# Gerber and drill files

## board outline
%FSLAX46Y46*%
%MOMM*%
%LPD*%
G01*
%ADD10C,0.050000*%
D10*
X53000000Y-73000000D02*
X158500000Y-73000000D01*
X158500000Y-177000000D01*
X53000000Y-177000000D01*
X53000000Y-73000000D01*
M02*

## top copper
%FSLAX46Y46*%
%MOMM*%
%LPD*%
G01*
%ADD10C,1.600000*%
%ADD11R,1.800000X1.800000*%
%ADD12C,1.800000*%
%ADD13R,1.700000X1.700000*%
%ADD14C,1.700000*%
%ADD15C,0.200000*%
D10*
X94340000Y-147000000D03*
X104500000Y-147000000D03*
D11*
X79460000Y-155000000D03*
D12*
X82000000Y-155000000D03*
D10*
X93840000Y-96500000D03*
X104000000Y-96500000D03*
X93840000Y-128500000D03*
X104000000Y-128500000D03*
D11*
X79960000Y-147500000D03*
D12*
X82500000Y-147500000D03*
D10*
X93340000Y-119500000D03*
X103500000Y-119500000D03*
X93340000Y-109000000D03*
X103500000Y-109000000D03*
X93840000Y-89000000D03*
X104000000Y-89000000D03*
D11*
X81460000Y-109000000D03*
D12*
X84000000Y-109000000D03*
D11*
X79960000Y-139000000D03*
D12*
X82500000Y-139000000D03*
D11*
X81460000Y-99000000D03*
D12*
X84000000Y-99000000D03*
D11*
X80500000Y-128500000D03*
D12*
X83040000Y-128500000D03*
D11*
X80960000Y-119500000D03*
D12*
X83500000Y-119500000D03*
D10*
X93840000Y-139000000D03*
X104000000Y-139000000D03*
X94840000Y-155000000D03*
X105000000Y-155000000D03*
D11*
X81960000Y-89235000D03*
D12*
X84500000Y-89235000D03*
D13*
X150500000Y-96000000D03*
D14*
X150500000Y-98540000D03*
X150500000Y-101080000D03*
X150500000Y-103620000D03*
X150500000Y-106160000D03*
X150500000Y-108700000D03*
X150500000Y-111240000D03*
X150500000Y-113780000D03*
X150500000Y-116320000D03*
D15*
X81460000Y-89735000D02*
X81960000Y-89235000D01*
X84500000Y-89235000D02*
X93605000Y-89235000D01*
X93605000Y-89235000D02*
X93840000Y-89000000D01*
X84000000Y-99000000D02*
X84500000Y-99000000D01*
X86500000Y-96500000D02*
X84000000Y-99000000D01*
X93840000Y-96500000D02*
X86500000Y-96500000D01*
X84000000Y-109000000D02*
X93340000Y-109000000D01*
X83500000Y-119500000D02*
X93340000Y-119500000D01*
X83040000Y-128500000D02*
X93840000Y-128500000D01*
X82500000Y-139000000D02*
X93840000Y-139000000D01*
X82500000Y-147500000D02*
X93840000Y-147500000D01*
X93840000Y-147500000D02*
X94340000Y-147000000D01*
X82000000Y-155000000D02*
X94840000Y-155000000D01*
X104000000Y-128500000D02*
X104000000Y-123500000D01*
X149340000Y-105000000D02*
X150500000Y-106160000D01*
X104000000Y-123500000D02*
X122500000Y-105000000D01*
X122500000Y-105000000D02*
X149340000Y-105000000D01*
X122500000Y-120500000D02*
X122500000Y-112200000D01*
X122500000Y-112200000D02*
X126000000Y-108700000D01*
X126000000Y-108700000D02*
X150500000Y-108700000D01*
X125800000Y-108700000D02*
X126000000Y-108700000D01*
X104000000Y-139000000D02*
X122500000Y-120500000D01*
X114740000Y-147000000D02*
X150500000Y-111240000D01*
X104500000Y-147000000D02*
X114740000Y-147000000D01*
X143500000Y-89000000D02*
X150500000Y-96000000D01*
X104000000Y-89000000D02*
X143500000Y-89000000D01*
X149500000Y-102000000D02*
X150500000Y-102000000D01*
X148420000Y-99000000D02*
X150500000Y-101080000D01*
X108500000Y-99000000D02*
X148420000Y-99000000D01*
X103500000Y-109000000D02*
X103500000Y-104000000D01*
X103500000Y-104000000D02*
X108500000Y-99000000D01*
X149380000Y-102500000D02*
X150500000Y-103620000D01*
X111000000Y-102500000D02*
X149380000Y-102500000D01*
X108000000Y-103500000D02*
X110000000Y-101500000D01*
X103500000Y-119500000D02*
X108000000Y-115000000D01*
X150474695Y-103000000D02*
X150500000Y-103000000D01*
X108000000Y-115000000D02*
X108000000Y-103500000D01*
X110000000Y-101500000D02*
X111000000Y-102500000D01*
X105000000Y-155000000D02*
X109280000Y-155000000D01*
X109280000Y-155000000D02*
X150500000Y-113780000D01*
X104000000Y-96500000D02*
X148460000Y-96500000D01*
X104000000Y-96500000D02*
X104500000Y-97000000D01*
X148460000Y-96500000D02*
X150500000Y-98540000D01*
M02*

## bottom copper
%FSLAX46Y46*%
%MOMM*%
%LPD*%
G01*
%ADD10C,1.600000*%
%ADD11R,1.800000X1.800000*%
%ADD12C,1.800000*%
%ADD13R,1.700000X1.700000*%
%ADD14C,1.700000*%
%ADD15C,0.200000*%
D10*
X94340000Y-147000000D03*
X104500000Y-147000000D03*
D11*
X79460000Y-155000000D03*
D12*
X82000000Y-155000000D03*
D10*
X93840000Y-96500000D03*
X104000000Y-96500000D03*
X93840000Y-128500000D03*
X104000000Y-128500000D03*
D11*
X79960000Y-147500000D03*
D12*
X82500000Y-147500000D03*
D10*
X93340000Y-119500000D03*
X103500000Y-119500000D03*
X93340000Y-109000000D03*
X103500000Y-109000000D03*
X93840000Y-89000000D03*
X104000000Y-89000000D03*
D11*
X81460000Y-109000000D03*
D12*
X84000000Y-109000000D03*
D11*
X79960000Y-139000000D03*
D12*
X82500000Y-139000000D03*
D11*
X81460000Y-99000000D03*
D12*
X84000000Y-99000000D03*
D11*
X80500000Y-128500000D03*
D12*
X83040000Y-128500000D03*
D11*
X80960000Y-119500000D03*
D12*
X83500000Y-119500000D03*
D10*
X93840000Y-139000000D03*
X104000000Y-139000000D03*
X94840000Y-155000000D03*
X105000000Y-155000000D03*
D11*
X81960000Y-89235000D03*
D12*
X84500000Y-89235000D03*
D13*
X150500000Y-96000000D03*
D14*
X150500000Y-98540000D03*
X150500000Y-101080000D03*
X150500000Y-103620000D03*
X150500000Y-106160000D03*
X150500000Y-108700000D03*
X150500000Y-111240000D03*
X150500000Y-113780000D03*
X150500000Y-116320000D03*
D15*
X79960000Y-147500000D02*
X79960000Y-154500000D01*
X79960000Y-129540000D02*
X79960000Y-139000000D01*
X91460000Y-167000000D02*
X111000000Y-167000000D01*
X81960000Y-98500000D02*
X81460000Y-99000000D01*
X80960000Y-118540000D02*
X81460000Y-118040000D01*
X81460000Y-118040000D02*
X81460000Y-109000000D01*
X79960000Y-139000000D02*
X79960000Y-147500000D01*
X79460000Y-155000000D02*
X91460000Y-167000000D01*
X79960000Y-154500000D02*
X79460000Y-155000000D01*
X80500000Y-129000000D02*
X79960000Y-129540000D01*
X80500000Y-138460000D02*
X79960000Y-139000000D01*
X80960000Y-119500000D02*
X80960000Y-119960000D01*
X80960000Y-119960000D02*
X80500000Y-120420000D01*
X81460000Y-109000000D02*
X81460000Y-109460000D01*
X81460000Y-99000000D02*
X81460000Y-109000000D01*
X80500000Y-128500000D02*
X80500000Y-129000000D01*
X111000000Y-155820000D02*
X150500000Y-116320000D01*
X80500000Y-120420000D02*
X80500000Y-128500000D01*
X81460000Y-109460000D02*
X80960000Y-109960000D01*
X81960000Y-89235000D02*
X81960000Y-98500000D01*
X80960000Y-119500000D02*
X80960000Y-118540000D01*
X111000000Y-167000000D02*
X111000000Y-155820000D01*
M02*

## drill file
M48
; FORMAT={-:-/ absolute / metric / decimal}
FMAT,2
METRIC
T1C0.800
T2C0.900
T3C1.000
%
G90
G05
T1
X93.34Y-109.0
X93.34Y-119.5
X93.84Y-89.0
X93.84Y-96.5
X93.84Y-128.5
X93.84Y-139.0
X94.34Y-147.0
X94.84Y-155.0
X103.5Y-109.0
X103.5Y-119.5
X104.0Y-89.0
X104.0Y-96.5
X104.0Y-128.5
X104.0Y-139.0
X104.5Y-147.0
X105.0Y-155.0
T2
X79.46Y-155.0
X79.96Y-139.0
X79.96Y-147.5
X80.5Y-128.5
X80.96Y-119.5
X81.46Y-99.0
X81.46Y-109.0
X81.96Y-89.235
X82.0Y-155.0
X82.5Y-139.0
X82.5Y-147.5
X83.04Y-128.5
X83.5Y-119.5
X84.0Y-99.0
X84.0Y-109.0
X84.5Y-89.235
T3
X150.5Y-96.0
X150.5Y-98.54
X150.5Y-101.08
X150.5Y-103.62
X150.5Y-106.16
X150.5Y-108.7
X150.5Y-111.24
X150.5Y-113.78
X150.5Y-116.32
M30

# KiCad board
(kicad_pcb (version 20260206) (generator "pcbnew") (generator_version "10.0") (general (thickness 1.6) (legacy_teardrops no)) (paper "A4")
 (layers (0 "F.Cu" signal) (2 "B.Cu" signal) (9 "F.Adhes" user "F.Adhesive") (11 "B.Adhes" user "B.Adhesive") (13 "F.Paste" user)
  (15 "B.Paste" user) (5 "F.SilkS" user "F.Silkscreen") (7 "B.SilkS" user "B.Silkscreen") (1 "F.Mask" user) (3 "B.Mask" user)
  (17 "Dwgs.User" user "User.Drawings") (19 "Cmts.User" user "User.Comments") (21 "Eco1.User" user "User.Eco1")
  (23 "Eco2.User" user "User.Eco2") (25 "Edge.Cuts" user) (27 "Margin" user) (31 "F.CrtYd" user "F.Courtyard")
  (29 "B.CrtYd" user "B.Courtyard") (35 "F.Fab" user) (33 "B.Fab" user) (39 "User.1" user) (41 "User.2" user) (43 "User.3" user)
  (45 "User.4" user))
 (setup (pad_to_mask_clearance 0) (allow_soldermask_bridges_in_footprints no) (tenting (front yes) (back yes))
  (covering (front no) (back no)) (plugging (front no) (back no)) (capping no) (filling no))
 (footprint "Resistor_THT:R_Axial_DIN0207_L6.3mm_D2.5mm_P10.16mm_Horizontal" (layer "F.Cu") (at 94.34 147)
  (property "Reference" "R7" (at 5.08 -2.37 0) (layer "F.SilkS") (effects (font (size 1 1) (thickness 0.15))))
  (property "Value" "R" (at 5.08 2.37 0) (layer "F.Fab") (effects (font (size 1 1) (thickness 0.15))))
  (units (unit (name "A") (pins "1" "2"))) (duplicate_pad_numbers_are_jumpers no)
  (pad "1" thru_hole circle (at 0 0) (size 1.6 1.6) (drill 0.8) (layers "*.Cu" "*.Mask") (remove_unused_layers no) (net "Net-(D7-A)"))
  (pad "2" thru_hole circle (at 10.16 0) (size 1.6 1.6) (drill 0.8) (layers "*.Cu" "*.Mask") (remove_unused_layers no)
   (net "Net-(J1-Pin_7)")))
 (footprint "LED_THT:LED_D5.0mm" (layer "F.Cu") (at 79.46 155)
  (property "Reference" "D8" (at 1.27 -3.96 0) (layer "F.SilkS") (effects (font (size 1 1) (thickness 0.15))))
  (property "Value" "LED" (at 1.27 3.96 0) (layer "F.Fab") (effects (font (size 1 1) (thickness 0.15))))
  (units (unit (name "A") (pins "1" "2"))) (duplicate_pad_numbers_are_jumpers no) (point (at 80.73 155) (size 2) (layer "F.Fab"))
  (pad "1" thru_hole rect (at 0 0) (size 1.8 1.8) (drill 0.9) (layers "*.Cu" "*.Mask") (remove_unused_layers no) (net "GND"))
  (pad "2" thru_hole circle (at 2.54 0) (size 1.8 1.8) (drill 0.9) (layers "*.Cu" "*.Mask") (remove_unused_layers no) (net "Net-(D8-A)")))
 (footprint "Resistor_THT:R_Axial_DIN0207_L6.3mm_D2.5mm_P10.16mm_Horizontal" (layer "F.Cu") (at 93.84 96.5)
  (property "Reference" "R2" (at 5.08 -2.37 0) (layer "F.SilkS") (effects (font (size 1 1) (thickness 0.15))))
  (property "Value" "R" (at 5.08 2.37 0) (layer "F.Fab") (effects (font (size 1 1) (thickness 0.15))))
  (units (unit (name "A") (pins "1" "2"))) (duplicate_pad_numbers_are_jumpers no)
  (pad "1" thru_hole circle (at 0 0) (size 1.6 1.6) (drill 0.8) (layers "*.Cu" "*.Mask") (remove_unused_layers no) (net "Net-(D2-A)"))
  (pad "2" thru_hole circle (at 10.16 0) (size 1.6 1.6) (drill 0.8) (layers "*.Cu" "*.Mask") (remove_unused_layers no)
   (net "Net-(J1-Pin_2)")))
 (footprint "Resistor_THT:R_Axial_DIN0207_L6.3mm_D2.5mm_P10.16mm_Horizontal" (layer "F.Cu") (at 93.84 128.5)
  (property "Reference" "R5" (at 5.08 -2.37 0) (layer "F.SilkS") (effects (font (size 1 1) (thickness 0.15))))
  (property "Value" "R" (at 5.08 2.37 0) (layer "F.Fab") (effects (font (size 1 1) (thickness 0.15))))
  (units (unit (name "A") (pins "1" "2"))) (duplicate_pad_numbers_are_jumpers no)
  (pad "1" thru_hole circle (at 0 0) (size 1.6 1.6) (drill 0.8) (layers "*.Cu" "*.Mask") (remove_unused_layers no) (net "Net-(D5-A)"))
  (pad "2" thru_hole circle (at 10.16 0) (size 1.6 1.6) (drill 0.8) (layers "*.Cu" "*.Mask") (remove_unused_layers no)
   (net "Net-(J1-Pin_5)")))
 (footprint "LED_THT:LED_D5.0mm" (layer "F.Cu") (at 79.96 147.5)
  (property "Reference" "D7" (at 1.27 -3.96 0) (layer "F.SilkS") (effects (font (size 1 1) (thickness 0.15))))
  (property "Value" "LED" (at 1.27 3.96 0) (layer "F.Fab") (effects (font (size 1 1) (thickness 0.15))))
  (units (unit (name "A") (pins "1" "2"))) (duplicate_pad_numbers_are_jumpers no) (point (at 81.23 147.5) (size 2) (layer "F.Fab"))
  (pad "1" thru_hole rect (at 0 0) (size 1.8 1.8) (drill 0.9) (layers "*.Cu" "*.Mask") (remove_unused_layers no) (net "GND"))
  (pad "2" thru_hole circle (at 2.54 0) (size 1.8 1.8) (drill 0.9) (layers "*.Cu" "*.Mask") (remove_unused_layers no) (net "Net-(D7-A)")))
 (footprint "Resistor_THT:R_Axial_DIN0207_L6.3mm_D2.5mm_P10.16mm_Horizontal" (layer "F.Cu") (at 93.34 119.5)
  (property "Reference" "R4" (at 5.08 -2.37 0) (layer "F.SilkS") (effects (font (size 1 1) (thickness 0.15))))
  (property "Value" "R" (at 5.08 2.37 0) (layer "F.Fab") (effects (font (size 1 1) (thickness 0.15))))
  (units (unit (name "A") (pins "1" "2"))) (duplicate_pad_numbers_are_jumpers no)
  (pad "1" thru_hole circle (at 0 0) (size 1.6 1.6) (drill 0.8) (layers "*.Cu" "*.Mask") (remove_unused_layers no) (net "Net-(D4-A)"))
  (pad "2" thru_hole circle (at 10.16 0) (size 1.6 1.6) (drill 0.8) (layers "*.Cu" "*.Mask") (remove_unused_layers no)
   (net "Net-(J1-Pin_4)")))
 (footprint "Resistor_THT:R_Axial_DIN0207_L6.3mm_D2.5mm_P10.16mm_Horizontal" (layer "F.Cu") (at 93.34 109)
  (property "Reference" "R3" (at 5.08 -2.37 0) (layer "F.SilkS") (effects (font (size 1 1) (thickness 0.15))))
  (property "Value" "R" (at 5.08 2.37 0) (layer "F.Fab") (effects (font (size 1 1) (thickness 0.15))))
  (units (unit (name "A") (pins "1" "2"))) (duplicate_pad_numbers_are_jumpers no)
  (pad "1" thru_hole circle (at 0 0) (size 1.6 1.6) (drill 0.8) (layers "*.Cu" "*.Mask") (remove_unused_layers no) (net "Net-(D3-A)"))
  (pad "2" thru_hole circle (at 10.16 0) (size 1.6 1.6) (drill 0.8) (layers "*.Cu" "*.Mask") (remove_unused_layers no)
   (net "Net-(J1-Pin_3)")))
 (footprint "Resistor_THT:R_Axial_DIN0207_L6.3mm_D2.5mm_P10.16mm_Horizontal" (layer "F.Cu") (at 93.84 89)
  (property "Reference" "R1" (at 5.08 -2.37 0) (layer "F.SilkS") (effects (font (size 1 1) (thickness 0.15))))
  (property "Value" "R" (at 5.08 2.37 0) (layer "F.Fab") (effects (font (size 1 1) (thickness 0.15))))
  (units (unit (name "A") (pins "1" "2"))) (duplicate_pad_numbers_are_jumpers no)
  (pad "1" thru_hole circle (at 0 0) (size 1.6 1.6) (drill 0.8) (layers "*.Cu" "*.Mask") (remove_unused_layers no) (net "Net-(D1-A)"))
  (pad "2" thru_hole circle (at 10.16 0) (size 1.6 1.6) (drill 0.8) (layers "*.Cu" "*.Mask") (remove_unused_layers no)
   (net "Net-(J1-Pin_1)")))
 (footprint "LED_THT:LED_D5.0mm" (layer "F.Cu") (at 81.46 109)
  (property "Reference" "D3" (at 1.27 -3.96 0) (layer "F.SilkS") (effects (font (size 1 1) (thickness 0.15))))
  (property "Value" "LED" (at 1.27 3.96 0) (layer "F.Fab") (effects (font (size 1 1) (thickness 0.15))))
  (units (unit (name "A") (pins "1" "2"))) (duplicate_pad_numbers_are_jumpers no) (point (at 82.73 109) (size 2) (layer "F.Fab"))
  (pad "1" thru_hole rect (at 0 0) (size 1.8 1.8) (drill 0.9) (layers "*.Cu" "*.Mask") (remove_unused_layers no) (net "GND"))
  (pad "2" thru_hole circle (at 2.54 0) (size 1.8 1.8) (drill 0.9) (layers "*.Cu" "*.Mask") (remove_unused_layers no) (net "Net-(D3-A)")))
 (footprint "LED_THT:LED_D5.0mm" (layer "F.Cu") (at 79.96 139)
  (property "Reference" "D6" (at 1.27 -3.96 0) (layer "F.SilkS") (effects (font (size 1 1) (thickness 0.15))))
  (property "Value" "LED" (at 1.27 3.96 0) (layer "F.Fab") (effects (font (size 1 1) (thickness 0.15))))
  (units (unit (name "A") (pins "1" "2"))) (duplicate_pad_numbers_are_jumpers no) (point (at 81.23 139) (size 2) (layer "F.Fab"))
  (pad "1" thru_hole rect (at 0 0) (size 1.8 1.8) (drill 0.9) (layers "*.Cu" "*.Mask") (remove_unused_layers no) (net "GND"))
  (pad "2" thru_hole circle (at 2.54 0) (size 1.8 1.8) (drill 0.9) (layers "*.Cu" "*.Mask") (remove_unused_layers no) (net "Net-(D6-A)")))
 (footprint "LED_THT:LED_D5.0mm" (layer "F.Cu") (at 81.46 99)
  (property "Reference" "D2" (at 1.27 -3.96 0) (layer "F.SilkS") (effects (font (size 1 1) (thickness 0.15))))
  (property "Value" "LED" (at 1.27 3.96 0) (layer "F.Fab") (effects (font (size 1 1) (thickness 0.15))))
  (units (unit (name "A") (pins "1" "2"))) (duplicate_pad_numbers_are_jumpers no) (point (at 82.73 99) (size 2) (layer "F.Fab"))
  (pad "1" thru_hole rect (at 0 0) (size 1.8 1.8) (drill 0.9) (layers "*.Cu" "*.Mask") (remove_unused_layers no) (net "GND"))
  (pad "2" thru_hole circle (at 2.54 0) (size 1.8 1.8) (drill 0.9) (layers "*.Cu" "*.Mask") (remove_unused_layers no) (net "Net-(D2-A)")))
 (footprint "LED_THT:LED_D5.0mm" (layer "F.Cu") (at 80.5 128.5)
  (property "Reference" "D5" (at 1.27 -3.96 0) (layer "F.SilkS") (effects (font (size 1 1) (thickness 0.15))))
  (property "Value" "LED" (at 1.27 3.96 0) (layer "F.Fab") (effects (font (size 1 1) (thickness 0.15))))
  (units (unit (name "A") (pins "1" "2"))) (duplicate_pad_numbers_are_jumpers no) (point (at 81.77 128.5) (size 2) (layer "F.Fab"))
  (pad "1" thru_hole rect (at 0 0) (size 1.8 1.8) (drill 0.9) (layers "*.Cu" "*.Mask") (remove_unused_layers no) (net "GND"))
  (pad "2" thru_hole circle (at 2.54 0) (size 1.8 1.8) (drill 0.9) (layers "*.Cu" "*.Mask") (remove_unused_layers no) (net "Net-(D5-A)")))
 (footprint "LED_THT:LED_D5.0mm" (layer "F.Cu") (at 80.96 119.5)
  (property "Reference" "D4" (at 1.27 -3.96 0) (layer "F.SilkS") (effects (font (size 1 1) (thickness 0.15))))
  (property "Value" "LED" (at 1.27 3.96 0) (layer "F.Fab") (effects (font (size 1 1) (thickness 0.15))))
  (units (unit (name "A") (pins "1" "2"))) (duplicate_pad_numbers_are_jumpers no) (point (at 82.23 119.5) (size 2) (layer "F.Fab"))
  (pad "1" thru_hole rect (at 0 0) (size 1.8 1.8) (drill 0.9) (layers "*.Cu" "*.Mask") (remove_unused_layers no) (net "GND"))
  (pad "2" thru_hole circle (at 2.54 0) (size 1.8 1.8) (drill 0.9) (layers "*.Cu" "*.Mask") (remove_unused_layers no) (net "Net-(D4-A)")))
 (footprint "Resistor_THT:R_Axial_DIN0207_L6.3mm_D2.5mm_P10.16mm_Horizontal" (layer "F.Cu") (at 93.84 139)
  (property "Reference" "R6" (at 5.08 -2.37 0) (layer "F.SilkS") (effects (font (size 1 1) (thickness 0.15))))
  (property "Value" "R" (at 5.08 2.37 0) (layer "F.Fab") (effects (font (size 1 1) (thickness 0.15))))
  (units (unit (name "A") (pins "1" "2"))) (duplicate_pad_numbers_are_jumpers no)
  (pad "1" thru_hole circle (at 0 0) (size 1.6 1.6) (drill 0.8) (layers "*.Cu" "*.Mask") (remove_unused_layers no) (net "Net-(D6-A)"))
  (pad "2" thru_hole circle (at 10.16 0) (size 1.6 1.6) (drill 0.8) (layers "*.Cu" "*.Mask") (remove_unused_layers no)
   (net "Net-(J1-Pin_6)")))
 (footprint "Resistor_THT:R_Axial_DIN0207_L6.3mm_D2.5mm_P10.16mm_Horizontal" (layer "F.Cu") (at 94.84 155)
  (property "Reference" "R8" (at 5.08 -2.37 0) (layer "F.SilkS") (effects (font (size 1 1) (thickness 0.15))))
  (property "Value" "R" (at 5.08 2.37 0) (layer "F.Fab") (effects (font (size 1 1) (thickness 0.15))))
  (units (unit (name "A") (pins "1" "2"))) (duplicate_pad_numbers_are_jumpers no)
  (pad "1" thru_hole circle (at 0 0) (size 1.6 1.6) (drill 0.8) (layers "*.Cu" "*.Mask") (remove_unused_layers no) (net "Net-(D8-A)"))
  (pad "2" thru_hole circle (at 10.16 0) (size 1.6 1.6) (drill 0.8) (layers "*.Cu" "*.Mask") (remove_unused_layers no)
   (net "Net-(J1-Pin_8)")))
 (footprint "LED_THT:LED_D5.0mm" (layer "F.Cu") (at 81.96 89.235)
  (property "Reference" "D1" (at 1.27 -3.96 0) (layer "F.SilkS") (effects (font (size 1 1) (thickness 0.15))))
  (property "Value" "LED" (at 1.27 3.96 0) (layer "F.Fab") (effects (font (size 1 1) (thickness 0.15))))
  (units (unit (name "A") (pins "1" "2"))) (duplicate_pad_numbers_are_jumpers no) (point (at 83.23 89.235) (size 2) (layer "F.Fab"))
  (pad "1" thru_hole rect (at 0 0) (size 1.8 1.8) (drill 0.9) (layers "*.Cu" "*.Mask") (remove_unused_layers no) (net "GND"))
  (pad "2" thru_hole circle (at 2.54 0) (size 1.8 1.8) (drill 0.9) (layers "*.Cu" "*.Mask") (remove_unused_layers no) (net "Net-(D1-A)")))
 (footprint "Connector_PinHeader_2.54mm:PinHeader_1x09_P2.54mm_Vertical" (layer "B.Cu") (at 150.5 96 180)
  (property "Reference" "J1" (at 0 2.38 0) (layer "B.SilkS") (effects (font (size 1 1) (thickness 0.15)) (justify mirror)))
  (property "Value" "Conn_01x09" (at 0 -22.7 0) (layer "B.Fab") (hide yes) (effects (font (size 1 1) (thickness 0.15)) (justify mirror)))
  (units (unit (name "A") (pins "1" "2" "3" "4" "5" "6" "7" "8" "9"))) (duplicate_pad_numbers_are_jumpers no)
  (pad "1" thru_hole rect (at 0 0 180) (size 1.7 1.7) (drill 1) (layers "*.Cu" "*.Mask") (remove_unused_layers no) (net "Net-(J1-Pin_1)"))
  (pad "2" thru_hole circle (at 0 -2.54 180) (size 1.7 1.7) (drill 1) (layers "*.Cu" "*.Mask") (remove_unused_layers no)
   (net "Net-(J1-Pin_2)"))
  (pad "3" thru_hole circle (at 0 -5.08 180) (size 1.7 1.7) (drill 1) (layers "*.Cu" "*.Mask") (remove_unused_layers no)
   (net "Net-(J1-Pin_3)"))
  (pad "4" thru_hole circle (at 0 -7.62 180) (size 1.7 1.7) (drill 1) (layers "*.Cu" "*.Mask") (remove_unused_layers no)
   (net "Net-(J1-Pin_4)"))
  (pad "5" thru_hole circle (at 0 -10.16 180) (size 1.7 1.7) (drill 1) (layers "*.Cu" "*.Mask") (remove_unused_layers no)
   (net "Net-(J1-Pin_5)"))
  (pad "6" thru_hole circle (at 0 -12.7 180) (size 1.7 1.7) (drill 1) (layers "*.Cu" "*.Mask") (remove_unused_layers no)
   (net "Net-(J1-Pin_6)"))
  (pad "7" thru_hole circle (at 0 -15.24 180) (size 1.7 1.7) (drill 1) (layers "*.Cu" "*.Mask") (remove_unused_layers no)
   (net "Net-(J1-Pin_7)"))
  (pad "8" thru_hole circle (at 0 -17.78 180) (size 1.7 1.7) (drill 1) (layers "*.Cu" "*.Mask") (remove_unused_layers no)
   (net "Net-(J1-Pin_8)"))
  (pad "9" thru_hole circle (at 0 -20.32 180) (size 1.7 1.7) (drill 1) (layers "*.Cu" "*.Mask") (remove_unused_layers no) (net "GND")))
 (gr_rect (start 53 73) (end 158.5 177) (stroke (width 0.05) (type default)) (fill no) (layer "Edge.Cuts"))
 (segment (start 81.46 89.735) (end 81.96 89.235) (width 0.2) (layer "F.Cu") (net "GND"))
 (segment (start 79.96 147.5) (end 79.96 154.5) (width 0.2) (layer "B.Cu") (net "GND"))
 (segment (start 79.96 129.54) (end 79.96 139) (width 0.2) (layer "B.Cu") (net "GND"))
 (segment (start 91.46 167) (end 111 167) (width 0.2) (layer "B.Cu") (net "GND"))
 (segment (start 81.96 98.5) (end 81.46 99) (width 0.2) (layer "B.Cu") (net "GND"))
 (segment (start 80.96 118.54) (end 81.46 118.04) (width 0.2) (layer "B.Cu") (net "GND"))
 (segment (start 81.46 118.04) (end 81.46 109) (width 0.2) (layer "B.Cu") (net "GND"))
 (segment (start 79.96 139) (end 79.96 147.5) (width 0.2) (layer "B.Cu") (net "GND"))
 (segment (start 79.46 155) (end 91.46 167) (width 0.2) (layer "B.Cu") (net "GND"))
 (segment (start 79.96 154.5) (end 79.46 155) (width 0.2) (layer "B.Cu") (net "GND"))
 (segment (start 80.5 129) (end 79.96 129.54) (width 0.2) (layer "B.Cu") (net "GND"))
 (segment (start 80.5 138.46) (end 79.96 139) (width 0.2) (layer "B.Cu") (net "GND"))
 (segment (start 80.96 119.5) (end 80.96 119.96) (width 0.2) (layer "B.Cu") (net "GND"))
 (segment (start 80.96 119.96) (end 80.5 120.42) (width 0.2) (layer "B.Cu") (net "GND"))
 (segment (start 81.46 109) (end 81.46 109.46) (width 0.2) (layer "B.Cu") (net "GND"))
 (segment (start 81.46 99) (end 81.46 109) (width 0.2) (layer "B.Cu") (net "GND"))
 (segment (start 80.5 128.5) (end 80.5 129) (width 0.2) (layer "B.Cu") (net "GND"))
 (segment (start 111 155.82) (end 150.5 116.32) (width 0.2) (layer "B.Cu") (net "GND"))
 (segment (start 80.5 120.42) (end 80.5 128.5) (width 0.2) (layer "B.Cu") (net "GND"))
 (segment (start 81.46 109.46) (end 80.96 109.96) (width 0.2) (layer "B.Cu") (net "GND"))
 (segment (start 81.96 89.235) (end 81.96 98.5) (width 0.2) (layer "B.Cu") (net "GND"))
 (segment (start 80.96 119.5) (end 80.96 118.54) (width 0.2) (layer "B.Cu") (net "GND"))
 (segment (start 111 167) (end 111 155.82) (width 0.2) (layer "B.Cu") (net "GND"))
 (segment (start 84.5 89.235) (end 93.605 89.235) (width 0.2) (layer "F.Cu") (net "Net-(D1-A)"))
 (segment (start 93.605 89.235) (end 93.84 89) (width 0.2) (layer "F.Cu") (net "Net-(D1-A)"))
 (segment (start 84 99) (end 84.5 99) (width 0.2) (layer "F.Cu") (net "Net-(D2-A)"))
 (segment (start 86.5 96.5) (end 84 99) (width 0.2) (layer "F.Cu") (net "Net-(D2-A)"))
 (segment (start 93.84 96.5) (end 86.5 96.5) (width 0.2) (layer "F.Cu") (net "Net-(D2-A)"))
 (segment (start 84 109) (end 93.34 109) (width 0.2) (layer "F.Cu") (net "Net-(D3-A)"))
 (segment (start 83.5 119.5) (end 93.34 119.5) (width 0.2) (layer "F.Cu") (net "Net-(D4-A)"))
 (segment (start 83.04 128.5) (end 93.84 128.5) (width 0.2) (layer "F.Cu") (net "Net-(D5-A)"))
 (segment (start 82.5 139) (end 93.84 139) (width 0.2) (layer "F.Cu") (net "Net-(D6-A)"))
 (segment (start 82.5 147.5) (end 93.84 147.5) (width 0.2) (layer "F.Cu") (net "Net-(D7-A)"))
 (segment (start 93.84 147.5) (end 94.34 147) (width 0.2) (layer "F.Cu") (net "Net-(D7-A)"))
 (segment (start 82 155) (end 94.84 155) (width 0.2) (layer "F.Cu") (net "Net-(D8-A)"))
 (segment (start 104 128.5) (end 104 123.5) (width 0.2) (layer "F.Cu") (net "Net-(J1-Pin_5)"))
 (segment (start 149.34 105) (end 150.5 106.16) (width 0.2) (layer "F.Cu") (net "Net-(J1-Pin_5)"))
 (segment (start 104 123.5) (end 122.5 105) (width 0.2) (layer "F.Cu") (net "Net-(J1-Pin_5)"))
 (segment (start 122.5 105) (end 149.34 105) (width 0.2) (layer "F.Cu") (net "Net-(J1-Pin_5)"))
 (segment (start 122.5 120.5) (end 122.5 112.2) (width 0.2) (layer "F.Cu") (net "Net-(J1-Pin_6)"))
 (segment (start 122.5 112.2) (end 126 108.7) (width 0.2) (layer "F.Cu") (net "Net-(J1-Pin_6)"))
 (segment (start 126 108.7) (end 150.5 108.7) (width 0.2) (layer "F.Cu") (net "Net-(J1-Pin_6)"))
 (segment (start 125.8 108.7) (end 126 108.7) (width 0.2) (layer "F.Cu") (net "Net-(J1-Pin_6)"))
 (segment (start 104 139) (end 122.5 120.5) (width 0.2) (layer "F.Cu") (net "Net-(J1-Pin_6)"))
 (segment (start 114.74 147) (end 150.5 111.24) (width 0.2) (layer "F.Cu") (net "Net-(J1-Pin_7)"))
 (segment (start 104.5 147) (end 114.74 147) (width 0.2) (layer "F.Cu") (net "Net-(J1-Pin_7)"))
 (segment (start 143.5 89) (end 150.5 96) (width 0.2) (layer "F.Cu") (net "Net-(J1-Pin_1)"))
 (segment (start 104 89) (end 143.5 89) (width 0.2) (layer "F.Cu") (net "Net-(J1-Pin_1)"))
 (segment (start 149.5 102) (end 150.5 102) (width 0.2) (layer "F.Cu") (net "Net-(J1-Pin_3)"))
 (segment (start 148.42 99) (end 150.5 101.08) (width 0.2) (layer "F.Cu") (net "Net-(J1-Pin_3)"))
 (segment (start 108.5 99) (end 148.42 99) (width 0.2) (layer "F.Cu") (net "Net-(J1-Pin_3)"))
 (segment (start 103.5 109) (end 103.5 104) (width 0.2) (layer "F.Cu") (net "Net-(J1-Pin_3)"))
 (segment (start 103.5 104) (end 108.5 99) (width 0.2) (layer "F.Cu") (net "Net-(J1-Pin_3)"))
 (segment (start 149.38 102.5) (end 150.5 103.62) (width 0.2) (layer "F.Cu") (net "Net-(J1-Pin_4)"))
 (segment (start 111 102.5) (end 149.38 102.5) (width 0.2) (layer "F.Cu") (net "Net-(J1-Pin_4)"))
 (segment (start 108 103.5) (end 110 101.5) (width 0.2) (layer "F.Cu") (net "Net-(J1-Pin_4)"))
 (segment (start 103.5 119.5) (end 108 115) (width 0.2) (layer "F.Cu") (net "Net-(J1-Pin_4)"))
 (segment (start 150.474695 103) (end 150.5 103) (width 0.2) (layer "F.Cu") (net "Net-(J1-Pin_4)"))
 (segment (start 108 115) (end 108 103.5) (width 0.2) (layer "F.Cu") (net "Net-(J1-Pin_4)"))
 (segment (start 110 101.5) (end 111 102.5) (width 0.2) (layer "F.Cu") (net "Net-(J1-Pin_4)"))
 (segment (start 105 155) (end 109.28 155) (width 0.2) (layer "F.Cu") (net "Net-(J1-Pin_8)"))
 (segment (start 109.28 155) (end 150.5 113.78) (width 0.2) (layer "F.Cu") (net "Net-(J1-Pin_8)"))
 (segment (start 104 96.5) (end 148.46 96.5) (width 0.2) (layer "F.Cu") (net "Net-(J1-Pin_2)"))
 (segment (start 104 96.5) (end 104.5 97) (width 0.2) (layer "F.Cu") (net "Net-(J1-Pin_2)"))
 (segment (start 148.46 96.5) (end 150.5 98.54) (width 0.2) (layer "F.Cu") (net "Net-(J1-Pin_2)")))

